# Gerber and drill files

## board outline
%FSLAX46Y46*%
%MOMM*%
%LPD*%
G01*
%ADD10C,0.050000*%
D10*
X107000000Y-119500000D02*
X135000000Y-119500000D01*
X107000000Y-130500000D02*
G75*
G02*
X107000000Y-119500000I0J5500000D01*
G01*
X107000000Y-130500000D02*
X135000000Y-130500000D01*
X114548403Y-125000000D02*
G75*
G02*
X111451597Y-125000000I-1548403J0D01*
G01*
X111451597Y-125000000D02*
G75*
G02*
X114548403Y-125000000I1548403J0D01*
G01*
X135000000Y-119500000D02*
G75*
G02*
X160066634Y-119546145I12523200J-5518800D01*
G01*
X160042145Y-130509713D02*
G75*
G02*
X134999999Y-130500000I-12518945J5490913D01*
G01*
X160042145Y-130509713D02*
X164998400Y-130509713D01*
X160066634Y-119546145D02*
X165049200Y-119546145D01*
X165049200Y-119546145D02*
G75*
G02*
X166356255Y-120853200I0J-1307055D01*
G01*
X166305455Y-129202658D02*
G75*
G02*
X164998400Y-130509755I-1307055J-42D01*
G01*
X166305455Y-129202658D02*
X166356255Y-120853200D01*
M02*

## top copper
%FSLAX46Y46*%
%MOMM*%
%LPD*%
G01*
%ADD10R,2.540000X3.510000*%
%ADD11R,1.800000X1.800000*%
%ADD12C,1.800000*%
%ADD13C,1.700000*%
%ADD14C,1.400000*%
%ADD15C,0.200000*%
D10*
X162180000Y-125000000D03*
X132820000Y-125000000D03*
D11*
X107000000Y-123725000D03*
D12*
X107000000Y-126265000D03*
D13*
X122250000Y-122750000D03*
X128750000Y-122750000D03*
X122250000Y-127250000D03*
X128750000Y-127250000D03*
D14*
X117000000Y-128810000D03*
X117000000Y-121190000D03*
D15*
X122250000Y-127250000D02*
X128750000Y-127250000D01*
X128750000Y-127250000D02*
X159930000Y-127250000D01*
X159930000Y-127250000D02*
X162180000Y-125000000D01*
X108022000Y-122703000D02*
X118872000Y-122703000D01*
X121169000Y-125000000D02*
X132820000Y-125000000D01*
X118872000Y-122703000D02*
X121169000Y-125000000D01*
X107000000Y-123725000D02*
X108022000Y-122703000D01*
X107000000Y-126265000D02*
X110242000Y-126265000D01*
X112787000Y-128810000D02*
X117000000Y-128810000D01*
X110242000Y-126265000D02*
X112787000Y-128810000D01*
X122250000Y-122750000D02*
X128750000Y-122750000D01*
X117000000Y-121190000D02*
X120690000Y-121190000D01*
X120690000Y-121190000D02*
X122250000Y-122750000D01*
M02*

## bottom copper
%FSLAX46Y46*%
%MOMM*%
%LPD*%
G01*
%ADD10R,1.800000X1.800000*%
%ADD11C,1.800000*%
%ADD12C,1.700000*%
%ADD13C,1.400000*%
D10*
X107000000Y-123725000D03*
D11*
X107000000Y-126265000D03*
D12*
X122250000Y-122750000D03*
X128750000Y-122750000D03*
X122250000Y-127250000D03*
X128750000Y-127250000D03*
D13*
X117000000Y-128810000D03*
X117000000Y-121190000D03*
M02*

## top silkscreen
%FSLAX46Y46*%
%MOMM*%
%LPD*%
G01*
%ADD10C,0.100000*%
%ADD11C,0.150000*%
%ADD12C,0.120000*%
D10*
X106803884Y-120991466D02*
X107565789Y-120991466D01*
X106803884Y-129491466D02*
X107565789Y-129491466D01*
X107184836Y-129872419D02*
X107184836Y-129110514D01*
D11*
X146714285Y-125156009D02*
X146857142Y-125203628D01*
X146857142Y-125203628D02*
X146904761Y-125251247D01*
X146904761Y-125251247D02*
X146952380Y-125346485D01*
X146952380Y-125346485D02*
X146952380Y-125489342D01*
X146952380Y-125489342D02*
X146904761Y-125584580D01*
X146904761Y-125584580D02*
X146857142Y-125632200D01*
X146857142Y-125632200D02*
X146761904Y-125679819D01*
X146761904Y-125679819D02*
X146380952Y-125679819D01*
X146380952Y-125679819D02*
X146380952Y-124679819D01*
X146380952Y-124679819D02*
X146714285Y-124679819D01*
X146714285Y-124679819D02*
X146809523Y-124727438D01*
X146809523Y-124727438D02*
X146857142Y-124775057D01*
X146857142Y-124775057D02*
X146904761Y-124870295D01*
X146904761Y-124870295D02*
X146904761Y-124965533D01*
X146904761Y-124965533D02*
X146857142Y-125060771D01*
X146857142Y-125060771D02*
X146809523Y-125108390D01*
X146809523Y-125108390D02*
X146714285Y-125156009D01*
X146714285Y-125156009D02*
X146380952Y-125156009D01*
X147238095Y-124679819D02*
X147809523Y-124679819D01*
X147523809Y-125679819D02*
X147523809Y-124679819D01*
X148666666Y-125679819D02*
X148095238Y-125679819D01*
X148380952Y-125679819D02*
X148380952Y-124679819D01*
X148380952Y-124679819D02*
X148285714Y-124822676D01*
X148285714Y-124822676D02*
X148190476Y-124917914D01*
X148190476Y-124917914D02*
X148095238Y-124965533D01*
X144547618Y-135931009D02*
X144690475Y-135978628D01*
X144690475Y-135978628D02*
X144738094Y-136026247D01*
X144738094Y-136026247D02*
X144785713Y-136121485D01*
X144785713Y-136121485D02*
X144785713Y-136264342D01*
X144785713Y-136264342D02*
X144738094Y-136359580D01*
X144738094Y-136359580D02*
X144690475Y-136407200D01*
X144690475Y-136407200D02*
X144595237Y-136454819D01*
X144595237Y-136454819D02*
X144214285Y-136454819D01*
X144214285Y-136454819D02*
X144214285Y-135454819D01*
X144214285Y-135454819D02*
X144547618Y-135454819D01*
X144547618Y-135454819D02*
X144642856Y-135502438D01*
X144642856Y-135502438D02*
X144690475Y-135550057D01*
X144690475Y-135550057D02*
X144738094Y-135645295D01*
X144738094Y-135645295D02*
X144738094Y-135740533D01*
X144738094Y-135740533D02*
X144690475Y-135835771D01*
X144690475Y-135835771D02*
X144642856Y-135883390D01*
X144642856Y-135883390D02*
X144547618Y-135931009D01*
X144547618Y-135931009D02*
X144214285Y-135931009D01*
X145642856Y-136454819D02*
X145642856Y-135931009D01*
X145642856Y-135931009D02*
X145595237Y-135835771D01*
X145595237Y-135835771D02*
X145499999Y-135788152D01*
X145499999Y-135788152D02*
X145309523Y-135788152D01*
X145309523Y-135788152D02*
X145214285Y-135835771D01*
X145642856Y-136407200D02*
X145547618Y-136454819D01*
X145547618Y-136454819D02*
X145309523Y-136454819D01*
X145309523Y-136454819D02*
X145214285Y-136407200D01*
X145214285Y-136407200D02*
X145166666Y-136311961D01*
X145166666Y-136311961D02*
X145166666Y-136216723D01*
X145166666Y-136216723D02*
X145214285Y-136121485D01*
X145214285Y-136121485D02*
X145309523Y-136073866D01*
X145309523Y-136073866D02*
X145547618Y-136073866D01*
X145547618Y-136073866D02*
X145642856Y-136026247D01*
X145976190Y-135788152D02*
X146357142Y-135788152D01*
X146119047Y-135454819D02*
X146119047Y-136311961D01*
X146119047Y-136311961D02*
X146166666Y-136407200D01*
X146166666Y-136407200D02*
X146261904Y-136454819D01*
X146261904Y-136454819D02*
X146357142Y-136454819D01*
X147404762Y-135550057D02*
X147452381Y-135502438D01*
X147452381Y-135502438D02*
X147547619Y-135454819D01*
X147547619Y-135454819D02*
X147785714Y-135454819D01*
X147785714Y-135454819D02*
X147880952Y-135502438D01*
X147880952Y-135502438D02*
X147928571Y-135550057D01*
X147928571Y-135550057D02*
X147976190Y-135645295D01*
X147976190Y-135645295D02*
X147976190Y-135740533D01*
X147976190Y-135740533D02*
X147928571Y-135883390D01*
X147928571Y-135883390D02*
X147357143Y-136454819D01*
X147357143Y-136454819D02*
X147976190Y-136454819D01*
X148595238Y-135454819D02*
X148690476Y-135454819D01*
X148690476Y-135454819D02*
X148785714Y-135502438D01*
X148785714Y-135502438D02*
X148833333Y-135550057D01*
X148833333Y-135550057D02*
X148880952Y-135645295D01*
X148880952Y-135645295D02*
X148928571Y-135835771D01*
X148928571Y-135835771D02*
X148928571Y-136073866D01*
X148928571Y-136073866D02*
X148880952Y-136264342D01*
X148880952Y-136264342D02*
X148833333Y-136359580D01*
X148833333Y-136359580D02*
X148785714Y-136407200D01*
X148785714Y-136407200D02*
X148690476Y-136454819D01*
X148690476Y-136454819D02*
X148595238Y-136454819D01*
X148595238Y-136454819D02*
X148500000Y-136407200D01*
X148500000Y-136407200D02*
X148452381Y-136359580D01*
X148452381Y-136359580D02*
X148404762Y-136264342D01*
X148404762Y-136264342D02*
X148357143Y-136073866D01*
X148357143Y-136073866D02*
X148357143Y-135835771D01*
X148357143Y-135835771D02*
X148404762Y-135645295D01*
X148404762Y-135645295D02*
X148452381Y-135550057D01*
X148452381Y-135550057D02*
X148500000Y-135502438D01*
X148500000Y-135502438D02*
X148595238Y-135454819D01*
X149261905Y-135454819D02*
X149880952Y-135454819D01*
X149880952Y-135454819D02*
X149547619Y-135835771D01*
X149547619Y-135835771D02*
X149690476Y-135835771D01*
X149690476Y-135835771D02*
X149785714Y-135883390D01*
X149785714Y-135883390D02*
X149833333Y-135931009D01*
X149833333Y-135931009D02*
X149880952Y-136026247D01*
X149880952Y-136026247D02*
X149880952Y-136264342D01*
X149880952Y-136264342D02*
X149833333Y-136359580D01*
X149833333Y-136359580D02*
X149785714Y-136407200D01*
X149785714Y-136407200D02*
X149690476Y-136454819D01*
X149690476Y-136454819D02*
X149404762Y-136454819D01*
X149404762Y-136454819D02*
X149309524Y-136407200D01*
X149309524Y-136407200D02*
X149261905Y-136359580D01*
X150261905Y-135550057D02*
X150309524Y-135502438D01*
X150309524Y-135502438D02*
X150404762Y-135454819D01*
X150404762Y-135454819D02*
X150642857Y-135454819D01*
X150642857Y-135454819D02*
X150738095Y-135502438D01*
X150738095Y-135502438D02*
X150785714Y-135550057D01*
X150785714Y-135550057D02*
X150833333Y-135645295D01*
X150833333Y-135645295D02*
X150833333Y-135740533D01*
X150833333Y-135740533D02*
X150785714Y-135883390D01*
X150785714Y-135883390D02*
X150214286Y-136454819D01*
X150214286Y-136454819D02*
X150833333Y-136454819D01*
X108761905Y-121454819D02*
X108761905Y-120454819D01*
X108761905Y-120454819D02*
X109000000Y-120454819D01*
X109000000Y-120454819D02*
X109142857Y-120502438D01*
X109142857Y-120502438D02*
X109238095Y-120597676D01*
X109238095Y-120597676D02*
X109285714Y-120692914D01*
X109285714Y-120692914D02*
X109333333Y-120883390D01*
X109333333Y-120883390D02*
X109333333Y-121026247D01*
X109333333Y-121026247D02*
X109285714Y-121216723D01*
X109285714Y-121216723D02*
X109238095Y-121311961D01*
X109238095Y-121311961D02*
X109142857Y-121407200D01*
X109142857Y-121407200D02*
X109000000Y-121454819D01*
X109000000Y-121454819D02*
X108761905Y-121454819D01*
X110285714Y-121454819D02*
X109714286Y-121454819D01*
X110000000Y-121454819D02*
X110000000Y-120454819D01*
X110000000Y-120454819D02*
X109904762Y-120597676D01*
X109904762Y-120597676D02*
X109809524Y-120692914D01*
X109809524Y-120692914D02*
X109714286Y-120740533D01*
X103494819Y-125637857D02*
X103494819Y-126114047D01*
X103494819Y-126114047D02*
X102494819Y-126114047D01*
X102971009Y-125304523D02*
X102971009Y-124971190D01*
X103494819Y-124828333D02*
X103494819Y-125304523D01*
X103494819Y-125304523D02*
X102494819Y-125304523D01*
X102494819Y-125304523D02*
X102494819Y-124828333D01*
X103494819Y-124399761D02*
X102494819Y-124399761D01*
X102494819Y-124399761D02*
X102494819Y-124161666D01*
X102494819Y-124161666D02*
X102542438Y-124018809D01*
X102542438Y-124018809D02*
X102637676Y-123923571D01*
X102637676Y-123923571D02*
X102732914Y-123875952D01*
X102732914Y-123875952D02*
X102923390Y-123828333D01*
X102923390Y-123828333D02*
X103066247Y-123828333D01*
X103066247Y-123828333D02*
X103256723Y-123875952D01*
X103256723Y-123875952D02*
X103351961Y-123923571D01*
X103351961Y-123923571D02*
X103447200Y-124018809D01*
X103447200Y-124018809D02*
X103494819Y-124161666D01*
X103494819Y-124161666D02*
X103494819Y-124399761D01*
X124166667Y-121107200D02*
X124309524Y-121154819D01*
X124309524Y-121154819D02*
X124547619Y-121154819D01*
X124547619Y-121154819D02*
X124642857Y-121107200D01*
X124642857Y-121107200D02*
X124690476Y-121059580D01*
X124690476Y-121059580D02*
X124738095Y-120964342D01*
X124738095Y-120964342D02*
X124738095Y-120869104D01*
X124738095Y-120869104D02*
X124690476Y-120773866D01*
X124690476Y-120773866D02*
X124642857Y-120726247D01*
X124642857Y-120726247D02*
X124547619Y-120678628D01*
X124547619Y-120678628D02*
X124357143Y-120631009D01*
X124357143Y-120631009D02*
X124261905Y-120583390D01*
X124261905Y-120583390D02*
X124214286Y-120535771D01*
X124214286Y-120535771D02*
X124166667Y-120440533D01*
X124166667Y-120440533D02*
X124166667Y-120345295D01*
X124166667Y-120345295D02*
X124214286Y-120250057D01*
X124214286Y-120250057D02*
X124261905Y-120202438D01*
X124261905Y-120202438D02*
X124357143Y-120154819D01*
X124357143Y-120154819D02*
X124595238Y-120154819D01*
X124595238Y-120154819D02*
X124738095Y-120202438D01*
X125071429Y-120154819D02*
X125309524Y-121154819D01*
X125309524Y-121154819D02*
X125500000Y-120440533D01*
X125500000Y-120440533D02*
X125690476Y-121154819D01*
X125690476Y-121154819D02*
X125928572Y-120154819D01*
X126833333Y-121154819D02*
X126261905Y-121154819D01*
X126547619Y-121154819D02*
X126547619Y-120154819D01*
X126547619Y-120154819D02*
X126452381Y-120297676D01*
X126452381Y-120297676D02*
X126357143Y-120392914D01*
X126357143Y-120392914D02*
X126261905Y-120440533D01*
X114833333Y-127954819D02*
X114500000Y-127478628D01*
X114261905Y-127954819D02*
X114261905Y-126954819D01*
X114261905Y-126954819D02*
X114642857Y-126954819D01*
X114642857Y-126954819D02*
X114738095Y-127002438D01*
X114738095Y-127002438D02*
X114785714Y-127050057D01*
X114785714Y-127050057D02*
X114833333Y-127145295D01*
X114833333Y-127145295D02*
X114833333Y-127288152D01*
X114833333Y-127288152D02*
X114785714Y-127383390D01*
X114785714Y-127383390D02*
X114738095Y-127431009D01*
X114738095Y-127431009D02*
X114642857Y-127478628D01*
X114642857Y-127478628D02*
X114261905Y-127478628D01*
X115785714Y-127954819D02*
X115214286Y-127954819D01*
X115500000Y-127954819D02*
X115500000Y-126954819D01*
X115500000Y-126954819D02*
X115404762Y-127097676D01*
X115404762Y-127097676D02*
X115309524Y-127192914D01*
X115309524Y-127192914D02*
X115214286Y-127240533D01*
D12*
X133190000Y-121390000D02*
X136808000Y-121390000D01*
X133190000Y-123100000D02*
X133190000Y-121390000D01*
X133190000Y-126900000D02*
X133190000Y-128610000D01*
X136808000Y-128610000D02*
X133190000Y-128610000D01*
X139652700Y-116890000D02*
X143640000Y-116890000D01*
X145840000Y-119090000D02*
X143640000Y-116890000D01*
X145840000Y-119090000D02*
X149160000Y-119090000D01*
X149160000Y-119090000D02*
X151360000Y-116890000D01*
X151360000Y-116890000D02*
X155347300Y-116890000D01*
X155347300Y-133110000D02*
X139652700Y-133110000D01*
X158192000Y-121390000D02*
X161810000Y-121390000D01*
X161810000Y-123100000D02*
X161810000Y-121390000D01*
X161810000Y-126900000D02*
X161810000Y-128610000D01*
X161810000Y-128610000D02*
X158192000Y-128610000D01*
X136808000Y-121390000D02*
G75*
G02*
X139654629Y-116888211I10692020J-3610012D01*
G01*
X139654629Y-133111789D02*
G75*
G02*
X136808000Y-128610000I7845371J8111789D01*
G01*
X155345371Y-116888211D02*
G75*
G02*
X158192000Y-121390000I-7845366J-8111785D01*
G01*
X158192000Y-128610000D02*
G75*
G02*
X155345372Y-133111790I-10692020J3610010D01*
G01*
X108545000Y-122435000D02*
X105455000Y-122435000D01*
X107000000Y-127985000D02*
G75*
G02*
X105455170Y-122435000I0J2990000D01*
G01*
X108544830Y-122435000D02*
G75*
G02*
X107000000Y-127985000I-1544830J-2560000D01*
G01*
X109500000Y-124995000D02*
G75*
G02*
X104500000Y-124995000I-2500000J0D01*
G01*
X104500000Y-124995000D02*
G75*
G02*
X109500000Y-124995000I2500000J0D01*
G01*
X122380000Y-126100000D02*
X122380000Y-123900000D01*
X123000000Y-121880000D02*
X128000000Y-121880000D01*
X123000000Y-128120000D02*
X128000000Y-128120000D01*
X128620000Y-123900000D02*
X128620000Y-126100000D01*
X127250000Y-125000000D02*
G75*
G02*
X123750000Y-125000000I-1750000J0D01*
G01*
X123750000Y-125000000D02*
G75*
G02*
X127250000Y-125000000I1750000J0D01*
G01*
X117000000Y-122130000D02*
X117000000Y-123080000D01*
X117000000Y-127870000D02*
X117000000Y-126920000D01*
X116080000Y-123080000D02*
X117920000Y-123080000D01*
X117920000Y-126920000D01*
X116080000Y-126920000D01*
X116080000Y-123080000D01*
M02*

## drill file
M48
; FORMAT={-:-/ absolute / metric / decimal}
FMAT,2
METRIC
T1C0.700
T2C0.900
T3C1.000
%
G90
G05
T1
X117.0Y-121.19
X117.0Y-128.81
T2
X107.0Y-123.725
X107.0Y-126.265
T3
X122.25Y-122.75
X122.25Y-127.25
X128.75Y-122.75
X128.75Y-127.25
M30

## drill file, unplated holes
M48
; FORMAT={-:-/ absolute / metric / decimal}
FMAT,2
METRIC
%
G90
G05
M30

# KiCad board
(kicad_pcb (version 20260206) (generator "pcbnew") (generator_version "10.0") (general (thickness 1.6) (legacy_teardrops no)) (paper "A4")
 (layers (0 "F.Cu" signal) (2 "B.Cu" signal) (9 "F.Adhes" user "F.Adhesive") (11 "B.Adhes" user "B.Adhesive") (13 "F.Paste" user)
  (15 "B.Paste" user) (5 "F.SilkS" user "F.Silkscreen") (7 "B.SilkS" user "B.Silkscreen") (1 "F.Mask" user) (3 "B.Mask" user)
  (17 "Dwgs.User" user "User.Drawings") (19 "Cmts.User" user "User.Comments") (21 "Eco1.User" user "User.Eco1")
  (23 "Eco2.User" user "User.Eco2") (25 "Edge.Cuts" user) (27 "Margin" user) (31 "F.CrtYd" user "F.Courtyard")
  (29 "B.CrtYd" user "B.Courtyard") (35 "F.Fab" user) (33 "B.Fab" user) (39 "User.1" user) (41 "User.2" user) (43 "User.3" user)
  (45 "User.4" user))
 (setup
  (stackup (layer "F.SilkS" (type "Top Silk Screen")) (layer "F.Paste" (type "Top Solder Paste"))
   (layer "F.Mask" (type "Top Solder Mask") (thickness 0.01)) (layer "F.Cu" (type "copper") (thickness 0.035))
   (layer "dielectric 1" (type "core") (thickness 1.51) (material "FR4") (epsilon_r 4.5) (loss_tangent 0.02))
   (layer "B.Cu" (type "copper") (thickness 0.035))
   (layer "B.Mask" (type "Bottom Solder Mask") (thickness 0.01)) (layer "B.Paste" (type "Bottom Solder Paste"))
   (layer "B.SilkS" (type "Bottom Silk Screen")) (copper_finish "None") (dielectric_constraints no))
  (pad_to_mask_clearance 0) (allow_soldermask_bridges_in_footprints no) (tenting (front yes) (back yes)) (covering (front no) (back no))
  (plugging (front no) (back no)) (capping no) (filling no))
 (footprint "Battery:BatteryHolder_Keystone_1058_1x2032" (layer "F.Cu") (at 147.5 125 180)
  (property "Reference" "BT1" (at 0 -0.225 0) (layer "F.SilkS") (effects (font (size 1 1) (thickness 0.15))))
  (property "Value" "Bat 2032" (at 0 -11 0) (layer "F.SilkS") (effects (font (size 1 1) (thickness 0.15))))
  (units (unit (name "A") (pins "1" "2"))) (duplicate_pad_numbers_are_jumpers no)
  (fp_line (start 14.31 3.61) (end 10.692 3.61) (stroke (width 0.12) (type solid)) (layer "F.SilkS"))
  (fp_line (start 14.31 1.9) (end 14.31 3.61) (stroke (width 0.12) (type solid)) (layer "F.SilkS"))
  (fp_line (start 14.31 -1.9) (end 14.31 -3.61) (stroke (width 0.12) (type solid)) (layer "F.SilkS"))
  (fp_line (start 10.692 -3.61) (end 14.31 -3.61) (stroke (width 0.12) (type solid)) (layer "F.SilkS"))
  (fp_line (start 7.8473 8.11) (end 3.86 8.11) (stroke (width 0.12) (type solid)) (layer "F.SilkS"))
  (fp_line (start 1.66 5.91) (end 3.86 8.11) (stroke (width 0.12) (type solid)) (layer "F.SilkS"))
  (fp_line (start 1.66 5.91) (end -1.66 5.91) (stroke (width 0.12) (type solid)) (layer "F.SilkS"))
  (fp_line (start -1.66 5.91) (end -3.86 8.11) (stroke (width 0.12) (type solid)) (layer "F.SilkS"))
  (fp_line (start -3.86 8.11) (end -7.8473 8.11) (stroke (width 0.12) (type solid)) (layer "F.SilkS"))
  (fp_line (start -7.8473 -8.11) (end 7.8473 -8.11) (stroke (width 0.12) (type solid)) (layer "F.SilkS"))
  (fp_line (start -10.692 3.61) (end -14.31 3.61) (stroke (width 0.12) (type solid)) (layer "F.SilkS"))
  (fp_line (start -14.31 1.9) (end -14.31 3.61) (stroke (width 0.12) (type solid)) (layer "F.SilkS"))
  (fp_line (start -14.31 -1.9) (end -14.31 -3.61) (stroke (width 0.12) (type solid)) (layer "F.SilkS"))
  (fp_line (start -14.31 -3.61) (end -10.692 -3.61) (stroke (width 0.12) (type solid)) (layer "F.SilkS"))
  (fp_arc (start 10.692 3.61) (mid 9.538084 6.031244) (end 7.845371 8.111789) (stroke (width 0.12) (type solid)) (layer "F.SilkS"))
  (fp_arc (start 7.845371 -8.111789) (mid 9.538085 -6.031244) (end 10.692 -3.61) (stroke (width 0.12) (type solid)) (layer "F.SilkS"))
  (fp_arc (start -7.845371 8.111789) (mid -9.538085 6.031244) (end -10.692 3.61) (stroke (width 0.12) (type solid)) (layer "F.SilkS"))
  (fp_arc (start -10.692 -3.61) (mid -9.538084 -6.031244) (end -7.845371 -8.111789) (stroke (width 0.12) (type solid)) (layer "F.SilkS"))
  (pad "1" smd rect (at -14.68 0 180) (size 2.54 3.51) (layers "F.Cu" "F.Mask" "F.Paste") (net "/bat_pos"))
  (pad "2" smd rect (at 14.68 0 180) (size 2.54 3.51) (layers "F.Cu" "F.Mask" "F.Paste") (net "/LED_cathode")))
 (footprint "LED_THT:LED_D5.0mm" (layer "F.Cu") (at 107 123.725 -90)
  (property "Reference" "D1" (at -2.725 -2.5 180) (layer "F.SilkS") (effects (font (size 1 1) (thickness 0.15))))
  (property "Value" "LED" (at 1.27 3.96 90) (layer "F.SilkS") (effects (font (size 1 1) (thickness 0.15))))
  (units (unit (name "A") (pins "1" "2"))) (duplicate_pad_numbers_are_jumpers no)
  (fp_line (start -1.29 -1.545) (end -1.29 1.545) (stroke (width 0.12) (type solid)) (layer "F.SilkS"))
  (fp_arc (start 4.26 0) (mid 2.071779 2.880495) (end -1.29 1.54483) (stroke (width 0.12) (type solid)) (layer "F.SilkS"))
  (fp_arc (start -1.29 -1.54483) (mid 2.071779 -2.880495) (end 4.26 0) (stroke (width 0.12) (type solid)) (layer "F.SilkS"))
  (fp_circle (center 1.27 0) (end 3.77 0) (stroke (width 0.12) (type solid)) (fill no) (layer "F.SilkS"))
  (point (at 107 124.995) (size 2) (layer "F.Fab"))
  (pad "1" thru_hole rect (at 0 0 270) (size 1.8 1.8) (drill 0.9) (layers "*.Cu" "*.Mask") (remove_unused_layers no) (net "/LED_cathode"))
  (pad "2" thru_hole circle (at 2.54 0 270) (size 1.8 1.8) (drill 0.9) (layers "*.Cu" "*.Mask") (remove_unused_layers no) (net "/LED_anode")))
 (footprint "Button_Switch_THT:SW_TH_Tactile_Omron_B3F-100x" (layer "F.Cu") (at 122.25 122.75)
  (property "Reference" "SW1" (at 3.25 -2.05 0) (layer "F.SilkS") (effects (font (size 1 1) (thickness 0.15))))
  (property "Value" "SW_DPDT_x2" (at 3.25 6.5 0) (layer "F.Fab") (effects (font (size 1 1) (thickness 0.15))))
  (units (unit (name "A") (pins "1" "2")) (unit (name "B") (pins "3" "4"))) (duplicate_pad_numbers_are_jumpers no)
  (fp_line (start 0.13 3.35) (end 0.13 1.15) (stroke (width 0.12) (type solid)) (layer "F.SilkS"))
  (fp_line (start 0.75 -0.87) (end 5.75 -0.87) (stroke (width 0.12) (type solid)) (layer "F.SilkS"))
  (fp_line (start 0.75 5.37) (end 5.75 5.37) (stroke (width 0.12) (type solid)) (layer "F.SilkS"))
  (fp_line (start 6.37 1.15) (end 6.37 3.35) (stroke (width 0.12) (type solid)) (layer "F.SilkS"))
  (fp_circle (center 3.25 2.25) (end 5 2.25) (stroke (width 0.12) (type solid)) (fill no) (layer "F.SilkS"))
  (pad "1" thru_hole circle (at 0 0) (size 1.7 1.7) (drill 1) (layers "*.Cu" "*.Mask") (remove_unused_layers no) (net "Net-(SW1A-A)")
   (thermal_bridge_angle 90))
  (pad "1" thru_hole circle (at 6.5 0) (size 1.7 1.7) (drill 1) (layers "*.Cu" "*.Mask") (remove_unused_layers no) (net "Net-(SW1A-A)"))
  (pad "2" thru_hole circle (at 0 4.5) (size 1.7 1.7) (drill 1) (layers "*.Cu" "*.Mask") (remove_unused_layers no) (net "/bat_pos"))
  (pad "2" thru_hole circle (at 6.5 4.5) (size 1.7 1.7) (drill 1) (layers "*.Cu" "*.Mask") (remove_unused_layers no) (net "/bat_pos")))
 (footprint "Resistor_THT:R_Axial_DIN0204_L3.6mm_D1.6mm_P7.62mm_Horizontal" (layer "F.Cu") (at 117 128.81 90)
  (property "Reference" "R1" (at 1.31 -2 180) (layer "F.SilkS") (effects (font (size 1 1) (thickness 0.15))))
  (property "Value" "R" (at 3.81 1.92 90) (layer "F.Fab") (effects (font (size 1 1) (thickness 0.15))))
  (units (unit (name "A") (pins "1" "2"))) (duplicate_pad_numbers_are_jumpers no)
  (fp_line (start 6.68 0) (end 5.73 0) (stroke (width 0.12) (type solid)) (layer "F.SilkS"))
  (fp_line (start 0.94 0) (end 1.89 0) (stroke (width 0.12) (type solid)) (layer "F.SilkS"))
  (fp_rect (start 1.89 -0.92) (end 5.73 0.92) (stroke (width 0.12) (type solid)) (fill no) (layer "F.SilkS"))
  (pad "1" thru_hole circle (at 0 0 90) (size 1.4 1.4) (drill 0.7) (layers "*.Cu" "*.Mask") (remove_unused_layers no) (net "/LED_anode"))
  (pad "2" thru_hole circle (at 7.62 0 90) (size 1.4 1.4) (drill 0.7) (layers "*.Cu" "*.Mask") (remove_unused_layers no)
   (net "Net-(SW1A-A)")))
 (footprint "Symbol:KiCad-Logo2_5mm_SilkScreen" (layer "B.Cu") (at 147.5 121.5 180)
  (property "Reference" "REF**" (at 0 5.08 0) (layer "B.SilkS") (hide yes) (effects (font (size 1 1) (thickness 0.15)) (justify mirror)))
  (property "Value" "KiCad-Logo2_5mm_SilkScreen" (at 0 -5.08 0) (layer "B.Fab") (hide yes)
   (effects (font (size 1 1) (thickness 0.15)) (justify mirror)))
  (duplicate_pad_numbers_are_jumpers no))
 (gr_line (start 107 119.5) (end 135 119.5) (stroke (width 0.05) (type default)) (locked yes) (layer "Edge.Cuts"))
 (gr_arc (start 107 130.5) (mid 101.5 125) (end 107 119.5) (stroke (width 0.05) (type default)) (locked yes) (layer "Edge.Cuts"))
 (gr_line (start 107 130.5) (end 135 130.5) (stroke (width 0.05) (type default)) (locked yes) (layer "Edge.Cuts"))
 (gr_circle (center 113 125) (end 113.1316 126.5428) (stroke (width 0.05) (type default)) (fill no) (layer "Edge.Cuts"))
 (gr_arc (start 135 119.5) (mid 147.548393 111.333514) (end 160.066634 119.546145) (stroke (width 0.05) (type default)) (locked yes)
  (layer "Edge.Cuts"))
 (gr_arc (start 160.042145 130.509713) (mid 147.517898 138.68899) (end 135 130.5) (stroke (width 0.05) (type default)) (locked yes)
  (layer "Edge.Cuts"))
 (gr_line (start 160.042145 130.509713) (end 164.9984 130.509713) (stroke (width 0.05) (type default)) (locked yes) (layer "Edge.Cuts"))
 (gr_line (start 160.066634 119.546145) (end 165.0492 119.546145) (stroke (width 0.05) (type default)) (locked yes) (layer "Edge.Cuts"))
 (gr_arc (start 165.0492 119.546145) (mid 165.973427 119.928973) (end 166.356255 120.8532) (stroke (width 0.05) (type default)) (locked yes)
  (layer "Edge.Cuts"))
 (gr_arc (start 166.305455 129.202658) (mid 165.922627 130.126885) (end 164.9984 130.509713) (stroke (width 0.05) (type default))
  (locked yes) (layer "Edge.Cuts"))
 (gr_line (start 166.305455 129.202658) (end 166.356255 120.8532) (stroke (width 0.05) (type default)) (locked yes) (layer "Edge.Cuts"))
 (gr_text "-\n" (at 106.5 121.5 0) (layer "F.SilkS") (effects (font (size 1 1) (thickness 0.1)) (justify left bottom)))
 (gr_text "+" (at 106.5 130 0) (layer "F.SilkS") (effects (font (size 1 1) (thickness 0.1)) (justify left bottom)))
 (segment (start 122.25 127.25) (end 128.75 127.25) (width 0.2) (layer "F.Cu") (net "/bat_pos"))
 (segment (start 128.75 127.25) (end 159.93 127.25) (width 0.2) (layer "F.Cu") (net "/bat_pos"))
 (segment (start 159.93 127.25) (end 162.18 125) (width 0.2) (layer "F.Cu") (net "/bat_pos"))
 (segment (start 108.022 122.703) (end 118.872 122.703) (width 0.2) (layer "F.Cu") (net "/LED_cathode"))
 (segment (start 121.169 125) (end 132.82 125) (width 0.2) (layer "F.Cu") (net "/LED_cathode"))
 (segment (start 118.872 122.703) (end 121.169 125) (width 0.2) (layer "F.Cu") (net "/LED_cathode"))
 (segment (start 107 123.725) (end 108.022 122.703) (width 0.2) (layer "F.Cu") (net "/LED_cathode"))
 (segment (start 107 126.265) (end 110.242 126.265) (width 0.2) (layer "F.Cu") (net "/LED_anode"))
 (segment (start 112.787 128.81) (end 117 128.81) (width 0.2) (layer "F.Cu") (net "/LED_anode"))
 (segment (start 110.242 126.265) (end 112.787 128.81) (width 0.2) (layer "F.Cu") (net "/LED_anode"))
 (segment (start 122.25 122.75) (end 128.75 122.75) (width 0.2) (layer "F.Cu") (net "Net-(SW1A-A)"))
 (segment (start 117 121.19) (end 120.69 121.19) (width 0.2) (layer "F.Cu") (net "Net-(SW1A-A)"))
 (segment (start 120.69 121.19) (end 122.25 122.75) (width 0.2) (layer "F.Cu") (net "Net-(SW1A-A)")))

